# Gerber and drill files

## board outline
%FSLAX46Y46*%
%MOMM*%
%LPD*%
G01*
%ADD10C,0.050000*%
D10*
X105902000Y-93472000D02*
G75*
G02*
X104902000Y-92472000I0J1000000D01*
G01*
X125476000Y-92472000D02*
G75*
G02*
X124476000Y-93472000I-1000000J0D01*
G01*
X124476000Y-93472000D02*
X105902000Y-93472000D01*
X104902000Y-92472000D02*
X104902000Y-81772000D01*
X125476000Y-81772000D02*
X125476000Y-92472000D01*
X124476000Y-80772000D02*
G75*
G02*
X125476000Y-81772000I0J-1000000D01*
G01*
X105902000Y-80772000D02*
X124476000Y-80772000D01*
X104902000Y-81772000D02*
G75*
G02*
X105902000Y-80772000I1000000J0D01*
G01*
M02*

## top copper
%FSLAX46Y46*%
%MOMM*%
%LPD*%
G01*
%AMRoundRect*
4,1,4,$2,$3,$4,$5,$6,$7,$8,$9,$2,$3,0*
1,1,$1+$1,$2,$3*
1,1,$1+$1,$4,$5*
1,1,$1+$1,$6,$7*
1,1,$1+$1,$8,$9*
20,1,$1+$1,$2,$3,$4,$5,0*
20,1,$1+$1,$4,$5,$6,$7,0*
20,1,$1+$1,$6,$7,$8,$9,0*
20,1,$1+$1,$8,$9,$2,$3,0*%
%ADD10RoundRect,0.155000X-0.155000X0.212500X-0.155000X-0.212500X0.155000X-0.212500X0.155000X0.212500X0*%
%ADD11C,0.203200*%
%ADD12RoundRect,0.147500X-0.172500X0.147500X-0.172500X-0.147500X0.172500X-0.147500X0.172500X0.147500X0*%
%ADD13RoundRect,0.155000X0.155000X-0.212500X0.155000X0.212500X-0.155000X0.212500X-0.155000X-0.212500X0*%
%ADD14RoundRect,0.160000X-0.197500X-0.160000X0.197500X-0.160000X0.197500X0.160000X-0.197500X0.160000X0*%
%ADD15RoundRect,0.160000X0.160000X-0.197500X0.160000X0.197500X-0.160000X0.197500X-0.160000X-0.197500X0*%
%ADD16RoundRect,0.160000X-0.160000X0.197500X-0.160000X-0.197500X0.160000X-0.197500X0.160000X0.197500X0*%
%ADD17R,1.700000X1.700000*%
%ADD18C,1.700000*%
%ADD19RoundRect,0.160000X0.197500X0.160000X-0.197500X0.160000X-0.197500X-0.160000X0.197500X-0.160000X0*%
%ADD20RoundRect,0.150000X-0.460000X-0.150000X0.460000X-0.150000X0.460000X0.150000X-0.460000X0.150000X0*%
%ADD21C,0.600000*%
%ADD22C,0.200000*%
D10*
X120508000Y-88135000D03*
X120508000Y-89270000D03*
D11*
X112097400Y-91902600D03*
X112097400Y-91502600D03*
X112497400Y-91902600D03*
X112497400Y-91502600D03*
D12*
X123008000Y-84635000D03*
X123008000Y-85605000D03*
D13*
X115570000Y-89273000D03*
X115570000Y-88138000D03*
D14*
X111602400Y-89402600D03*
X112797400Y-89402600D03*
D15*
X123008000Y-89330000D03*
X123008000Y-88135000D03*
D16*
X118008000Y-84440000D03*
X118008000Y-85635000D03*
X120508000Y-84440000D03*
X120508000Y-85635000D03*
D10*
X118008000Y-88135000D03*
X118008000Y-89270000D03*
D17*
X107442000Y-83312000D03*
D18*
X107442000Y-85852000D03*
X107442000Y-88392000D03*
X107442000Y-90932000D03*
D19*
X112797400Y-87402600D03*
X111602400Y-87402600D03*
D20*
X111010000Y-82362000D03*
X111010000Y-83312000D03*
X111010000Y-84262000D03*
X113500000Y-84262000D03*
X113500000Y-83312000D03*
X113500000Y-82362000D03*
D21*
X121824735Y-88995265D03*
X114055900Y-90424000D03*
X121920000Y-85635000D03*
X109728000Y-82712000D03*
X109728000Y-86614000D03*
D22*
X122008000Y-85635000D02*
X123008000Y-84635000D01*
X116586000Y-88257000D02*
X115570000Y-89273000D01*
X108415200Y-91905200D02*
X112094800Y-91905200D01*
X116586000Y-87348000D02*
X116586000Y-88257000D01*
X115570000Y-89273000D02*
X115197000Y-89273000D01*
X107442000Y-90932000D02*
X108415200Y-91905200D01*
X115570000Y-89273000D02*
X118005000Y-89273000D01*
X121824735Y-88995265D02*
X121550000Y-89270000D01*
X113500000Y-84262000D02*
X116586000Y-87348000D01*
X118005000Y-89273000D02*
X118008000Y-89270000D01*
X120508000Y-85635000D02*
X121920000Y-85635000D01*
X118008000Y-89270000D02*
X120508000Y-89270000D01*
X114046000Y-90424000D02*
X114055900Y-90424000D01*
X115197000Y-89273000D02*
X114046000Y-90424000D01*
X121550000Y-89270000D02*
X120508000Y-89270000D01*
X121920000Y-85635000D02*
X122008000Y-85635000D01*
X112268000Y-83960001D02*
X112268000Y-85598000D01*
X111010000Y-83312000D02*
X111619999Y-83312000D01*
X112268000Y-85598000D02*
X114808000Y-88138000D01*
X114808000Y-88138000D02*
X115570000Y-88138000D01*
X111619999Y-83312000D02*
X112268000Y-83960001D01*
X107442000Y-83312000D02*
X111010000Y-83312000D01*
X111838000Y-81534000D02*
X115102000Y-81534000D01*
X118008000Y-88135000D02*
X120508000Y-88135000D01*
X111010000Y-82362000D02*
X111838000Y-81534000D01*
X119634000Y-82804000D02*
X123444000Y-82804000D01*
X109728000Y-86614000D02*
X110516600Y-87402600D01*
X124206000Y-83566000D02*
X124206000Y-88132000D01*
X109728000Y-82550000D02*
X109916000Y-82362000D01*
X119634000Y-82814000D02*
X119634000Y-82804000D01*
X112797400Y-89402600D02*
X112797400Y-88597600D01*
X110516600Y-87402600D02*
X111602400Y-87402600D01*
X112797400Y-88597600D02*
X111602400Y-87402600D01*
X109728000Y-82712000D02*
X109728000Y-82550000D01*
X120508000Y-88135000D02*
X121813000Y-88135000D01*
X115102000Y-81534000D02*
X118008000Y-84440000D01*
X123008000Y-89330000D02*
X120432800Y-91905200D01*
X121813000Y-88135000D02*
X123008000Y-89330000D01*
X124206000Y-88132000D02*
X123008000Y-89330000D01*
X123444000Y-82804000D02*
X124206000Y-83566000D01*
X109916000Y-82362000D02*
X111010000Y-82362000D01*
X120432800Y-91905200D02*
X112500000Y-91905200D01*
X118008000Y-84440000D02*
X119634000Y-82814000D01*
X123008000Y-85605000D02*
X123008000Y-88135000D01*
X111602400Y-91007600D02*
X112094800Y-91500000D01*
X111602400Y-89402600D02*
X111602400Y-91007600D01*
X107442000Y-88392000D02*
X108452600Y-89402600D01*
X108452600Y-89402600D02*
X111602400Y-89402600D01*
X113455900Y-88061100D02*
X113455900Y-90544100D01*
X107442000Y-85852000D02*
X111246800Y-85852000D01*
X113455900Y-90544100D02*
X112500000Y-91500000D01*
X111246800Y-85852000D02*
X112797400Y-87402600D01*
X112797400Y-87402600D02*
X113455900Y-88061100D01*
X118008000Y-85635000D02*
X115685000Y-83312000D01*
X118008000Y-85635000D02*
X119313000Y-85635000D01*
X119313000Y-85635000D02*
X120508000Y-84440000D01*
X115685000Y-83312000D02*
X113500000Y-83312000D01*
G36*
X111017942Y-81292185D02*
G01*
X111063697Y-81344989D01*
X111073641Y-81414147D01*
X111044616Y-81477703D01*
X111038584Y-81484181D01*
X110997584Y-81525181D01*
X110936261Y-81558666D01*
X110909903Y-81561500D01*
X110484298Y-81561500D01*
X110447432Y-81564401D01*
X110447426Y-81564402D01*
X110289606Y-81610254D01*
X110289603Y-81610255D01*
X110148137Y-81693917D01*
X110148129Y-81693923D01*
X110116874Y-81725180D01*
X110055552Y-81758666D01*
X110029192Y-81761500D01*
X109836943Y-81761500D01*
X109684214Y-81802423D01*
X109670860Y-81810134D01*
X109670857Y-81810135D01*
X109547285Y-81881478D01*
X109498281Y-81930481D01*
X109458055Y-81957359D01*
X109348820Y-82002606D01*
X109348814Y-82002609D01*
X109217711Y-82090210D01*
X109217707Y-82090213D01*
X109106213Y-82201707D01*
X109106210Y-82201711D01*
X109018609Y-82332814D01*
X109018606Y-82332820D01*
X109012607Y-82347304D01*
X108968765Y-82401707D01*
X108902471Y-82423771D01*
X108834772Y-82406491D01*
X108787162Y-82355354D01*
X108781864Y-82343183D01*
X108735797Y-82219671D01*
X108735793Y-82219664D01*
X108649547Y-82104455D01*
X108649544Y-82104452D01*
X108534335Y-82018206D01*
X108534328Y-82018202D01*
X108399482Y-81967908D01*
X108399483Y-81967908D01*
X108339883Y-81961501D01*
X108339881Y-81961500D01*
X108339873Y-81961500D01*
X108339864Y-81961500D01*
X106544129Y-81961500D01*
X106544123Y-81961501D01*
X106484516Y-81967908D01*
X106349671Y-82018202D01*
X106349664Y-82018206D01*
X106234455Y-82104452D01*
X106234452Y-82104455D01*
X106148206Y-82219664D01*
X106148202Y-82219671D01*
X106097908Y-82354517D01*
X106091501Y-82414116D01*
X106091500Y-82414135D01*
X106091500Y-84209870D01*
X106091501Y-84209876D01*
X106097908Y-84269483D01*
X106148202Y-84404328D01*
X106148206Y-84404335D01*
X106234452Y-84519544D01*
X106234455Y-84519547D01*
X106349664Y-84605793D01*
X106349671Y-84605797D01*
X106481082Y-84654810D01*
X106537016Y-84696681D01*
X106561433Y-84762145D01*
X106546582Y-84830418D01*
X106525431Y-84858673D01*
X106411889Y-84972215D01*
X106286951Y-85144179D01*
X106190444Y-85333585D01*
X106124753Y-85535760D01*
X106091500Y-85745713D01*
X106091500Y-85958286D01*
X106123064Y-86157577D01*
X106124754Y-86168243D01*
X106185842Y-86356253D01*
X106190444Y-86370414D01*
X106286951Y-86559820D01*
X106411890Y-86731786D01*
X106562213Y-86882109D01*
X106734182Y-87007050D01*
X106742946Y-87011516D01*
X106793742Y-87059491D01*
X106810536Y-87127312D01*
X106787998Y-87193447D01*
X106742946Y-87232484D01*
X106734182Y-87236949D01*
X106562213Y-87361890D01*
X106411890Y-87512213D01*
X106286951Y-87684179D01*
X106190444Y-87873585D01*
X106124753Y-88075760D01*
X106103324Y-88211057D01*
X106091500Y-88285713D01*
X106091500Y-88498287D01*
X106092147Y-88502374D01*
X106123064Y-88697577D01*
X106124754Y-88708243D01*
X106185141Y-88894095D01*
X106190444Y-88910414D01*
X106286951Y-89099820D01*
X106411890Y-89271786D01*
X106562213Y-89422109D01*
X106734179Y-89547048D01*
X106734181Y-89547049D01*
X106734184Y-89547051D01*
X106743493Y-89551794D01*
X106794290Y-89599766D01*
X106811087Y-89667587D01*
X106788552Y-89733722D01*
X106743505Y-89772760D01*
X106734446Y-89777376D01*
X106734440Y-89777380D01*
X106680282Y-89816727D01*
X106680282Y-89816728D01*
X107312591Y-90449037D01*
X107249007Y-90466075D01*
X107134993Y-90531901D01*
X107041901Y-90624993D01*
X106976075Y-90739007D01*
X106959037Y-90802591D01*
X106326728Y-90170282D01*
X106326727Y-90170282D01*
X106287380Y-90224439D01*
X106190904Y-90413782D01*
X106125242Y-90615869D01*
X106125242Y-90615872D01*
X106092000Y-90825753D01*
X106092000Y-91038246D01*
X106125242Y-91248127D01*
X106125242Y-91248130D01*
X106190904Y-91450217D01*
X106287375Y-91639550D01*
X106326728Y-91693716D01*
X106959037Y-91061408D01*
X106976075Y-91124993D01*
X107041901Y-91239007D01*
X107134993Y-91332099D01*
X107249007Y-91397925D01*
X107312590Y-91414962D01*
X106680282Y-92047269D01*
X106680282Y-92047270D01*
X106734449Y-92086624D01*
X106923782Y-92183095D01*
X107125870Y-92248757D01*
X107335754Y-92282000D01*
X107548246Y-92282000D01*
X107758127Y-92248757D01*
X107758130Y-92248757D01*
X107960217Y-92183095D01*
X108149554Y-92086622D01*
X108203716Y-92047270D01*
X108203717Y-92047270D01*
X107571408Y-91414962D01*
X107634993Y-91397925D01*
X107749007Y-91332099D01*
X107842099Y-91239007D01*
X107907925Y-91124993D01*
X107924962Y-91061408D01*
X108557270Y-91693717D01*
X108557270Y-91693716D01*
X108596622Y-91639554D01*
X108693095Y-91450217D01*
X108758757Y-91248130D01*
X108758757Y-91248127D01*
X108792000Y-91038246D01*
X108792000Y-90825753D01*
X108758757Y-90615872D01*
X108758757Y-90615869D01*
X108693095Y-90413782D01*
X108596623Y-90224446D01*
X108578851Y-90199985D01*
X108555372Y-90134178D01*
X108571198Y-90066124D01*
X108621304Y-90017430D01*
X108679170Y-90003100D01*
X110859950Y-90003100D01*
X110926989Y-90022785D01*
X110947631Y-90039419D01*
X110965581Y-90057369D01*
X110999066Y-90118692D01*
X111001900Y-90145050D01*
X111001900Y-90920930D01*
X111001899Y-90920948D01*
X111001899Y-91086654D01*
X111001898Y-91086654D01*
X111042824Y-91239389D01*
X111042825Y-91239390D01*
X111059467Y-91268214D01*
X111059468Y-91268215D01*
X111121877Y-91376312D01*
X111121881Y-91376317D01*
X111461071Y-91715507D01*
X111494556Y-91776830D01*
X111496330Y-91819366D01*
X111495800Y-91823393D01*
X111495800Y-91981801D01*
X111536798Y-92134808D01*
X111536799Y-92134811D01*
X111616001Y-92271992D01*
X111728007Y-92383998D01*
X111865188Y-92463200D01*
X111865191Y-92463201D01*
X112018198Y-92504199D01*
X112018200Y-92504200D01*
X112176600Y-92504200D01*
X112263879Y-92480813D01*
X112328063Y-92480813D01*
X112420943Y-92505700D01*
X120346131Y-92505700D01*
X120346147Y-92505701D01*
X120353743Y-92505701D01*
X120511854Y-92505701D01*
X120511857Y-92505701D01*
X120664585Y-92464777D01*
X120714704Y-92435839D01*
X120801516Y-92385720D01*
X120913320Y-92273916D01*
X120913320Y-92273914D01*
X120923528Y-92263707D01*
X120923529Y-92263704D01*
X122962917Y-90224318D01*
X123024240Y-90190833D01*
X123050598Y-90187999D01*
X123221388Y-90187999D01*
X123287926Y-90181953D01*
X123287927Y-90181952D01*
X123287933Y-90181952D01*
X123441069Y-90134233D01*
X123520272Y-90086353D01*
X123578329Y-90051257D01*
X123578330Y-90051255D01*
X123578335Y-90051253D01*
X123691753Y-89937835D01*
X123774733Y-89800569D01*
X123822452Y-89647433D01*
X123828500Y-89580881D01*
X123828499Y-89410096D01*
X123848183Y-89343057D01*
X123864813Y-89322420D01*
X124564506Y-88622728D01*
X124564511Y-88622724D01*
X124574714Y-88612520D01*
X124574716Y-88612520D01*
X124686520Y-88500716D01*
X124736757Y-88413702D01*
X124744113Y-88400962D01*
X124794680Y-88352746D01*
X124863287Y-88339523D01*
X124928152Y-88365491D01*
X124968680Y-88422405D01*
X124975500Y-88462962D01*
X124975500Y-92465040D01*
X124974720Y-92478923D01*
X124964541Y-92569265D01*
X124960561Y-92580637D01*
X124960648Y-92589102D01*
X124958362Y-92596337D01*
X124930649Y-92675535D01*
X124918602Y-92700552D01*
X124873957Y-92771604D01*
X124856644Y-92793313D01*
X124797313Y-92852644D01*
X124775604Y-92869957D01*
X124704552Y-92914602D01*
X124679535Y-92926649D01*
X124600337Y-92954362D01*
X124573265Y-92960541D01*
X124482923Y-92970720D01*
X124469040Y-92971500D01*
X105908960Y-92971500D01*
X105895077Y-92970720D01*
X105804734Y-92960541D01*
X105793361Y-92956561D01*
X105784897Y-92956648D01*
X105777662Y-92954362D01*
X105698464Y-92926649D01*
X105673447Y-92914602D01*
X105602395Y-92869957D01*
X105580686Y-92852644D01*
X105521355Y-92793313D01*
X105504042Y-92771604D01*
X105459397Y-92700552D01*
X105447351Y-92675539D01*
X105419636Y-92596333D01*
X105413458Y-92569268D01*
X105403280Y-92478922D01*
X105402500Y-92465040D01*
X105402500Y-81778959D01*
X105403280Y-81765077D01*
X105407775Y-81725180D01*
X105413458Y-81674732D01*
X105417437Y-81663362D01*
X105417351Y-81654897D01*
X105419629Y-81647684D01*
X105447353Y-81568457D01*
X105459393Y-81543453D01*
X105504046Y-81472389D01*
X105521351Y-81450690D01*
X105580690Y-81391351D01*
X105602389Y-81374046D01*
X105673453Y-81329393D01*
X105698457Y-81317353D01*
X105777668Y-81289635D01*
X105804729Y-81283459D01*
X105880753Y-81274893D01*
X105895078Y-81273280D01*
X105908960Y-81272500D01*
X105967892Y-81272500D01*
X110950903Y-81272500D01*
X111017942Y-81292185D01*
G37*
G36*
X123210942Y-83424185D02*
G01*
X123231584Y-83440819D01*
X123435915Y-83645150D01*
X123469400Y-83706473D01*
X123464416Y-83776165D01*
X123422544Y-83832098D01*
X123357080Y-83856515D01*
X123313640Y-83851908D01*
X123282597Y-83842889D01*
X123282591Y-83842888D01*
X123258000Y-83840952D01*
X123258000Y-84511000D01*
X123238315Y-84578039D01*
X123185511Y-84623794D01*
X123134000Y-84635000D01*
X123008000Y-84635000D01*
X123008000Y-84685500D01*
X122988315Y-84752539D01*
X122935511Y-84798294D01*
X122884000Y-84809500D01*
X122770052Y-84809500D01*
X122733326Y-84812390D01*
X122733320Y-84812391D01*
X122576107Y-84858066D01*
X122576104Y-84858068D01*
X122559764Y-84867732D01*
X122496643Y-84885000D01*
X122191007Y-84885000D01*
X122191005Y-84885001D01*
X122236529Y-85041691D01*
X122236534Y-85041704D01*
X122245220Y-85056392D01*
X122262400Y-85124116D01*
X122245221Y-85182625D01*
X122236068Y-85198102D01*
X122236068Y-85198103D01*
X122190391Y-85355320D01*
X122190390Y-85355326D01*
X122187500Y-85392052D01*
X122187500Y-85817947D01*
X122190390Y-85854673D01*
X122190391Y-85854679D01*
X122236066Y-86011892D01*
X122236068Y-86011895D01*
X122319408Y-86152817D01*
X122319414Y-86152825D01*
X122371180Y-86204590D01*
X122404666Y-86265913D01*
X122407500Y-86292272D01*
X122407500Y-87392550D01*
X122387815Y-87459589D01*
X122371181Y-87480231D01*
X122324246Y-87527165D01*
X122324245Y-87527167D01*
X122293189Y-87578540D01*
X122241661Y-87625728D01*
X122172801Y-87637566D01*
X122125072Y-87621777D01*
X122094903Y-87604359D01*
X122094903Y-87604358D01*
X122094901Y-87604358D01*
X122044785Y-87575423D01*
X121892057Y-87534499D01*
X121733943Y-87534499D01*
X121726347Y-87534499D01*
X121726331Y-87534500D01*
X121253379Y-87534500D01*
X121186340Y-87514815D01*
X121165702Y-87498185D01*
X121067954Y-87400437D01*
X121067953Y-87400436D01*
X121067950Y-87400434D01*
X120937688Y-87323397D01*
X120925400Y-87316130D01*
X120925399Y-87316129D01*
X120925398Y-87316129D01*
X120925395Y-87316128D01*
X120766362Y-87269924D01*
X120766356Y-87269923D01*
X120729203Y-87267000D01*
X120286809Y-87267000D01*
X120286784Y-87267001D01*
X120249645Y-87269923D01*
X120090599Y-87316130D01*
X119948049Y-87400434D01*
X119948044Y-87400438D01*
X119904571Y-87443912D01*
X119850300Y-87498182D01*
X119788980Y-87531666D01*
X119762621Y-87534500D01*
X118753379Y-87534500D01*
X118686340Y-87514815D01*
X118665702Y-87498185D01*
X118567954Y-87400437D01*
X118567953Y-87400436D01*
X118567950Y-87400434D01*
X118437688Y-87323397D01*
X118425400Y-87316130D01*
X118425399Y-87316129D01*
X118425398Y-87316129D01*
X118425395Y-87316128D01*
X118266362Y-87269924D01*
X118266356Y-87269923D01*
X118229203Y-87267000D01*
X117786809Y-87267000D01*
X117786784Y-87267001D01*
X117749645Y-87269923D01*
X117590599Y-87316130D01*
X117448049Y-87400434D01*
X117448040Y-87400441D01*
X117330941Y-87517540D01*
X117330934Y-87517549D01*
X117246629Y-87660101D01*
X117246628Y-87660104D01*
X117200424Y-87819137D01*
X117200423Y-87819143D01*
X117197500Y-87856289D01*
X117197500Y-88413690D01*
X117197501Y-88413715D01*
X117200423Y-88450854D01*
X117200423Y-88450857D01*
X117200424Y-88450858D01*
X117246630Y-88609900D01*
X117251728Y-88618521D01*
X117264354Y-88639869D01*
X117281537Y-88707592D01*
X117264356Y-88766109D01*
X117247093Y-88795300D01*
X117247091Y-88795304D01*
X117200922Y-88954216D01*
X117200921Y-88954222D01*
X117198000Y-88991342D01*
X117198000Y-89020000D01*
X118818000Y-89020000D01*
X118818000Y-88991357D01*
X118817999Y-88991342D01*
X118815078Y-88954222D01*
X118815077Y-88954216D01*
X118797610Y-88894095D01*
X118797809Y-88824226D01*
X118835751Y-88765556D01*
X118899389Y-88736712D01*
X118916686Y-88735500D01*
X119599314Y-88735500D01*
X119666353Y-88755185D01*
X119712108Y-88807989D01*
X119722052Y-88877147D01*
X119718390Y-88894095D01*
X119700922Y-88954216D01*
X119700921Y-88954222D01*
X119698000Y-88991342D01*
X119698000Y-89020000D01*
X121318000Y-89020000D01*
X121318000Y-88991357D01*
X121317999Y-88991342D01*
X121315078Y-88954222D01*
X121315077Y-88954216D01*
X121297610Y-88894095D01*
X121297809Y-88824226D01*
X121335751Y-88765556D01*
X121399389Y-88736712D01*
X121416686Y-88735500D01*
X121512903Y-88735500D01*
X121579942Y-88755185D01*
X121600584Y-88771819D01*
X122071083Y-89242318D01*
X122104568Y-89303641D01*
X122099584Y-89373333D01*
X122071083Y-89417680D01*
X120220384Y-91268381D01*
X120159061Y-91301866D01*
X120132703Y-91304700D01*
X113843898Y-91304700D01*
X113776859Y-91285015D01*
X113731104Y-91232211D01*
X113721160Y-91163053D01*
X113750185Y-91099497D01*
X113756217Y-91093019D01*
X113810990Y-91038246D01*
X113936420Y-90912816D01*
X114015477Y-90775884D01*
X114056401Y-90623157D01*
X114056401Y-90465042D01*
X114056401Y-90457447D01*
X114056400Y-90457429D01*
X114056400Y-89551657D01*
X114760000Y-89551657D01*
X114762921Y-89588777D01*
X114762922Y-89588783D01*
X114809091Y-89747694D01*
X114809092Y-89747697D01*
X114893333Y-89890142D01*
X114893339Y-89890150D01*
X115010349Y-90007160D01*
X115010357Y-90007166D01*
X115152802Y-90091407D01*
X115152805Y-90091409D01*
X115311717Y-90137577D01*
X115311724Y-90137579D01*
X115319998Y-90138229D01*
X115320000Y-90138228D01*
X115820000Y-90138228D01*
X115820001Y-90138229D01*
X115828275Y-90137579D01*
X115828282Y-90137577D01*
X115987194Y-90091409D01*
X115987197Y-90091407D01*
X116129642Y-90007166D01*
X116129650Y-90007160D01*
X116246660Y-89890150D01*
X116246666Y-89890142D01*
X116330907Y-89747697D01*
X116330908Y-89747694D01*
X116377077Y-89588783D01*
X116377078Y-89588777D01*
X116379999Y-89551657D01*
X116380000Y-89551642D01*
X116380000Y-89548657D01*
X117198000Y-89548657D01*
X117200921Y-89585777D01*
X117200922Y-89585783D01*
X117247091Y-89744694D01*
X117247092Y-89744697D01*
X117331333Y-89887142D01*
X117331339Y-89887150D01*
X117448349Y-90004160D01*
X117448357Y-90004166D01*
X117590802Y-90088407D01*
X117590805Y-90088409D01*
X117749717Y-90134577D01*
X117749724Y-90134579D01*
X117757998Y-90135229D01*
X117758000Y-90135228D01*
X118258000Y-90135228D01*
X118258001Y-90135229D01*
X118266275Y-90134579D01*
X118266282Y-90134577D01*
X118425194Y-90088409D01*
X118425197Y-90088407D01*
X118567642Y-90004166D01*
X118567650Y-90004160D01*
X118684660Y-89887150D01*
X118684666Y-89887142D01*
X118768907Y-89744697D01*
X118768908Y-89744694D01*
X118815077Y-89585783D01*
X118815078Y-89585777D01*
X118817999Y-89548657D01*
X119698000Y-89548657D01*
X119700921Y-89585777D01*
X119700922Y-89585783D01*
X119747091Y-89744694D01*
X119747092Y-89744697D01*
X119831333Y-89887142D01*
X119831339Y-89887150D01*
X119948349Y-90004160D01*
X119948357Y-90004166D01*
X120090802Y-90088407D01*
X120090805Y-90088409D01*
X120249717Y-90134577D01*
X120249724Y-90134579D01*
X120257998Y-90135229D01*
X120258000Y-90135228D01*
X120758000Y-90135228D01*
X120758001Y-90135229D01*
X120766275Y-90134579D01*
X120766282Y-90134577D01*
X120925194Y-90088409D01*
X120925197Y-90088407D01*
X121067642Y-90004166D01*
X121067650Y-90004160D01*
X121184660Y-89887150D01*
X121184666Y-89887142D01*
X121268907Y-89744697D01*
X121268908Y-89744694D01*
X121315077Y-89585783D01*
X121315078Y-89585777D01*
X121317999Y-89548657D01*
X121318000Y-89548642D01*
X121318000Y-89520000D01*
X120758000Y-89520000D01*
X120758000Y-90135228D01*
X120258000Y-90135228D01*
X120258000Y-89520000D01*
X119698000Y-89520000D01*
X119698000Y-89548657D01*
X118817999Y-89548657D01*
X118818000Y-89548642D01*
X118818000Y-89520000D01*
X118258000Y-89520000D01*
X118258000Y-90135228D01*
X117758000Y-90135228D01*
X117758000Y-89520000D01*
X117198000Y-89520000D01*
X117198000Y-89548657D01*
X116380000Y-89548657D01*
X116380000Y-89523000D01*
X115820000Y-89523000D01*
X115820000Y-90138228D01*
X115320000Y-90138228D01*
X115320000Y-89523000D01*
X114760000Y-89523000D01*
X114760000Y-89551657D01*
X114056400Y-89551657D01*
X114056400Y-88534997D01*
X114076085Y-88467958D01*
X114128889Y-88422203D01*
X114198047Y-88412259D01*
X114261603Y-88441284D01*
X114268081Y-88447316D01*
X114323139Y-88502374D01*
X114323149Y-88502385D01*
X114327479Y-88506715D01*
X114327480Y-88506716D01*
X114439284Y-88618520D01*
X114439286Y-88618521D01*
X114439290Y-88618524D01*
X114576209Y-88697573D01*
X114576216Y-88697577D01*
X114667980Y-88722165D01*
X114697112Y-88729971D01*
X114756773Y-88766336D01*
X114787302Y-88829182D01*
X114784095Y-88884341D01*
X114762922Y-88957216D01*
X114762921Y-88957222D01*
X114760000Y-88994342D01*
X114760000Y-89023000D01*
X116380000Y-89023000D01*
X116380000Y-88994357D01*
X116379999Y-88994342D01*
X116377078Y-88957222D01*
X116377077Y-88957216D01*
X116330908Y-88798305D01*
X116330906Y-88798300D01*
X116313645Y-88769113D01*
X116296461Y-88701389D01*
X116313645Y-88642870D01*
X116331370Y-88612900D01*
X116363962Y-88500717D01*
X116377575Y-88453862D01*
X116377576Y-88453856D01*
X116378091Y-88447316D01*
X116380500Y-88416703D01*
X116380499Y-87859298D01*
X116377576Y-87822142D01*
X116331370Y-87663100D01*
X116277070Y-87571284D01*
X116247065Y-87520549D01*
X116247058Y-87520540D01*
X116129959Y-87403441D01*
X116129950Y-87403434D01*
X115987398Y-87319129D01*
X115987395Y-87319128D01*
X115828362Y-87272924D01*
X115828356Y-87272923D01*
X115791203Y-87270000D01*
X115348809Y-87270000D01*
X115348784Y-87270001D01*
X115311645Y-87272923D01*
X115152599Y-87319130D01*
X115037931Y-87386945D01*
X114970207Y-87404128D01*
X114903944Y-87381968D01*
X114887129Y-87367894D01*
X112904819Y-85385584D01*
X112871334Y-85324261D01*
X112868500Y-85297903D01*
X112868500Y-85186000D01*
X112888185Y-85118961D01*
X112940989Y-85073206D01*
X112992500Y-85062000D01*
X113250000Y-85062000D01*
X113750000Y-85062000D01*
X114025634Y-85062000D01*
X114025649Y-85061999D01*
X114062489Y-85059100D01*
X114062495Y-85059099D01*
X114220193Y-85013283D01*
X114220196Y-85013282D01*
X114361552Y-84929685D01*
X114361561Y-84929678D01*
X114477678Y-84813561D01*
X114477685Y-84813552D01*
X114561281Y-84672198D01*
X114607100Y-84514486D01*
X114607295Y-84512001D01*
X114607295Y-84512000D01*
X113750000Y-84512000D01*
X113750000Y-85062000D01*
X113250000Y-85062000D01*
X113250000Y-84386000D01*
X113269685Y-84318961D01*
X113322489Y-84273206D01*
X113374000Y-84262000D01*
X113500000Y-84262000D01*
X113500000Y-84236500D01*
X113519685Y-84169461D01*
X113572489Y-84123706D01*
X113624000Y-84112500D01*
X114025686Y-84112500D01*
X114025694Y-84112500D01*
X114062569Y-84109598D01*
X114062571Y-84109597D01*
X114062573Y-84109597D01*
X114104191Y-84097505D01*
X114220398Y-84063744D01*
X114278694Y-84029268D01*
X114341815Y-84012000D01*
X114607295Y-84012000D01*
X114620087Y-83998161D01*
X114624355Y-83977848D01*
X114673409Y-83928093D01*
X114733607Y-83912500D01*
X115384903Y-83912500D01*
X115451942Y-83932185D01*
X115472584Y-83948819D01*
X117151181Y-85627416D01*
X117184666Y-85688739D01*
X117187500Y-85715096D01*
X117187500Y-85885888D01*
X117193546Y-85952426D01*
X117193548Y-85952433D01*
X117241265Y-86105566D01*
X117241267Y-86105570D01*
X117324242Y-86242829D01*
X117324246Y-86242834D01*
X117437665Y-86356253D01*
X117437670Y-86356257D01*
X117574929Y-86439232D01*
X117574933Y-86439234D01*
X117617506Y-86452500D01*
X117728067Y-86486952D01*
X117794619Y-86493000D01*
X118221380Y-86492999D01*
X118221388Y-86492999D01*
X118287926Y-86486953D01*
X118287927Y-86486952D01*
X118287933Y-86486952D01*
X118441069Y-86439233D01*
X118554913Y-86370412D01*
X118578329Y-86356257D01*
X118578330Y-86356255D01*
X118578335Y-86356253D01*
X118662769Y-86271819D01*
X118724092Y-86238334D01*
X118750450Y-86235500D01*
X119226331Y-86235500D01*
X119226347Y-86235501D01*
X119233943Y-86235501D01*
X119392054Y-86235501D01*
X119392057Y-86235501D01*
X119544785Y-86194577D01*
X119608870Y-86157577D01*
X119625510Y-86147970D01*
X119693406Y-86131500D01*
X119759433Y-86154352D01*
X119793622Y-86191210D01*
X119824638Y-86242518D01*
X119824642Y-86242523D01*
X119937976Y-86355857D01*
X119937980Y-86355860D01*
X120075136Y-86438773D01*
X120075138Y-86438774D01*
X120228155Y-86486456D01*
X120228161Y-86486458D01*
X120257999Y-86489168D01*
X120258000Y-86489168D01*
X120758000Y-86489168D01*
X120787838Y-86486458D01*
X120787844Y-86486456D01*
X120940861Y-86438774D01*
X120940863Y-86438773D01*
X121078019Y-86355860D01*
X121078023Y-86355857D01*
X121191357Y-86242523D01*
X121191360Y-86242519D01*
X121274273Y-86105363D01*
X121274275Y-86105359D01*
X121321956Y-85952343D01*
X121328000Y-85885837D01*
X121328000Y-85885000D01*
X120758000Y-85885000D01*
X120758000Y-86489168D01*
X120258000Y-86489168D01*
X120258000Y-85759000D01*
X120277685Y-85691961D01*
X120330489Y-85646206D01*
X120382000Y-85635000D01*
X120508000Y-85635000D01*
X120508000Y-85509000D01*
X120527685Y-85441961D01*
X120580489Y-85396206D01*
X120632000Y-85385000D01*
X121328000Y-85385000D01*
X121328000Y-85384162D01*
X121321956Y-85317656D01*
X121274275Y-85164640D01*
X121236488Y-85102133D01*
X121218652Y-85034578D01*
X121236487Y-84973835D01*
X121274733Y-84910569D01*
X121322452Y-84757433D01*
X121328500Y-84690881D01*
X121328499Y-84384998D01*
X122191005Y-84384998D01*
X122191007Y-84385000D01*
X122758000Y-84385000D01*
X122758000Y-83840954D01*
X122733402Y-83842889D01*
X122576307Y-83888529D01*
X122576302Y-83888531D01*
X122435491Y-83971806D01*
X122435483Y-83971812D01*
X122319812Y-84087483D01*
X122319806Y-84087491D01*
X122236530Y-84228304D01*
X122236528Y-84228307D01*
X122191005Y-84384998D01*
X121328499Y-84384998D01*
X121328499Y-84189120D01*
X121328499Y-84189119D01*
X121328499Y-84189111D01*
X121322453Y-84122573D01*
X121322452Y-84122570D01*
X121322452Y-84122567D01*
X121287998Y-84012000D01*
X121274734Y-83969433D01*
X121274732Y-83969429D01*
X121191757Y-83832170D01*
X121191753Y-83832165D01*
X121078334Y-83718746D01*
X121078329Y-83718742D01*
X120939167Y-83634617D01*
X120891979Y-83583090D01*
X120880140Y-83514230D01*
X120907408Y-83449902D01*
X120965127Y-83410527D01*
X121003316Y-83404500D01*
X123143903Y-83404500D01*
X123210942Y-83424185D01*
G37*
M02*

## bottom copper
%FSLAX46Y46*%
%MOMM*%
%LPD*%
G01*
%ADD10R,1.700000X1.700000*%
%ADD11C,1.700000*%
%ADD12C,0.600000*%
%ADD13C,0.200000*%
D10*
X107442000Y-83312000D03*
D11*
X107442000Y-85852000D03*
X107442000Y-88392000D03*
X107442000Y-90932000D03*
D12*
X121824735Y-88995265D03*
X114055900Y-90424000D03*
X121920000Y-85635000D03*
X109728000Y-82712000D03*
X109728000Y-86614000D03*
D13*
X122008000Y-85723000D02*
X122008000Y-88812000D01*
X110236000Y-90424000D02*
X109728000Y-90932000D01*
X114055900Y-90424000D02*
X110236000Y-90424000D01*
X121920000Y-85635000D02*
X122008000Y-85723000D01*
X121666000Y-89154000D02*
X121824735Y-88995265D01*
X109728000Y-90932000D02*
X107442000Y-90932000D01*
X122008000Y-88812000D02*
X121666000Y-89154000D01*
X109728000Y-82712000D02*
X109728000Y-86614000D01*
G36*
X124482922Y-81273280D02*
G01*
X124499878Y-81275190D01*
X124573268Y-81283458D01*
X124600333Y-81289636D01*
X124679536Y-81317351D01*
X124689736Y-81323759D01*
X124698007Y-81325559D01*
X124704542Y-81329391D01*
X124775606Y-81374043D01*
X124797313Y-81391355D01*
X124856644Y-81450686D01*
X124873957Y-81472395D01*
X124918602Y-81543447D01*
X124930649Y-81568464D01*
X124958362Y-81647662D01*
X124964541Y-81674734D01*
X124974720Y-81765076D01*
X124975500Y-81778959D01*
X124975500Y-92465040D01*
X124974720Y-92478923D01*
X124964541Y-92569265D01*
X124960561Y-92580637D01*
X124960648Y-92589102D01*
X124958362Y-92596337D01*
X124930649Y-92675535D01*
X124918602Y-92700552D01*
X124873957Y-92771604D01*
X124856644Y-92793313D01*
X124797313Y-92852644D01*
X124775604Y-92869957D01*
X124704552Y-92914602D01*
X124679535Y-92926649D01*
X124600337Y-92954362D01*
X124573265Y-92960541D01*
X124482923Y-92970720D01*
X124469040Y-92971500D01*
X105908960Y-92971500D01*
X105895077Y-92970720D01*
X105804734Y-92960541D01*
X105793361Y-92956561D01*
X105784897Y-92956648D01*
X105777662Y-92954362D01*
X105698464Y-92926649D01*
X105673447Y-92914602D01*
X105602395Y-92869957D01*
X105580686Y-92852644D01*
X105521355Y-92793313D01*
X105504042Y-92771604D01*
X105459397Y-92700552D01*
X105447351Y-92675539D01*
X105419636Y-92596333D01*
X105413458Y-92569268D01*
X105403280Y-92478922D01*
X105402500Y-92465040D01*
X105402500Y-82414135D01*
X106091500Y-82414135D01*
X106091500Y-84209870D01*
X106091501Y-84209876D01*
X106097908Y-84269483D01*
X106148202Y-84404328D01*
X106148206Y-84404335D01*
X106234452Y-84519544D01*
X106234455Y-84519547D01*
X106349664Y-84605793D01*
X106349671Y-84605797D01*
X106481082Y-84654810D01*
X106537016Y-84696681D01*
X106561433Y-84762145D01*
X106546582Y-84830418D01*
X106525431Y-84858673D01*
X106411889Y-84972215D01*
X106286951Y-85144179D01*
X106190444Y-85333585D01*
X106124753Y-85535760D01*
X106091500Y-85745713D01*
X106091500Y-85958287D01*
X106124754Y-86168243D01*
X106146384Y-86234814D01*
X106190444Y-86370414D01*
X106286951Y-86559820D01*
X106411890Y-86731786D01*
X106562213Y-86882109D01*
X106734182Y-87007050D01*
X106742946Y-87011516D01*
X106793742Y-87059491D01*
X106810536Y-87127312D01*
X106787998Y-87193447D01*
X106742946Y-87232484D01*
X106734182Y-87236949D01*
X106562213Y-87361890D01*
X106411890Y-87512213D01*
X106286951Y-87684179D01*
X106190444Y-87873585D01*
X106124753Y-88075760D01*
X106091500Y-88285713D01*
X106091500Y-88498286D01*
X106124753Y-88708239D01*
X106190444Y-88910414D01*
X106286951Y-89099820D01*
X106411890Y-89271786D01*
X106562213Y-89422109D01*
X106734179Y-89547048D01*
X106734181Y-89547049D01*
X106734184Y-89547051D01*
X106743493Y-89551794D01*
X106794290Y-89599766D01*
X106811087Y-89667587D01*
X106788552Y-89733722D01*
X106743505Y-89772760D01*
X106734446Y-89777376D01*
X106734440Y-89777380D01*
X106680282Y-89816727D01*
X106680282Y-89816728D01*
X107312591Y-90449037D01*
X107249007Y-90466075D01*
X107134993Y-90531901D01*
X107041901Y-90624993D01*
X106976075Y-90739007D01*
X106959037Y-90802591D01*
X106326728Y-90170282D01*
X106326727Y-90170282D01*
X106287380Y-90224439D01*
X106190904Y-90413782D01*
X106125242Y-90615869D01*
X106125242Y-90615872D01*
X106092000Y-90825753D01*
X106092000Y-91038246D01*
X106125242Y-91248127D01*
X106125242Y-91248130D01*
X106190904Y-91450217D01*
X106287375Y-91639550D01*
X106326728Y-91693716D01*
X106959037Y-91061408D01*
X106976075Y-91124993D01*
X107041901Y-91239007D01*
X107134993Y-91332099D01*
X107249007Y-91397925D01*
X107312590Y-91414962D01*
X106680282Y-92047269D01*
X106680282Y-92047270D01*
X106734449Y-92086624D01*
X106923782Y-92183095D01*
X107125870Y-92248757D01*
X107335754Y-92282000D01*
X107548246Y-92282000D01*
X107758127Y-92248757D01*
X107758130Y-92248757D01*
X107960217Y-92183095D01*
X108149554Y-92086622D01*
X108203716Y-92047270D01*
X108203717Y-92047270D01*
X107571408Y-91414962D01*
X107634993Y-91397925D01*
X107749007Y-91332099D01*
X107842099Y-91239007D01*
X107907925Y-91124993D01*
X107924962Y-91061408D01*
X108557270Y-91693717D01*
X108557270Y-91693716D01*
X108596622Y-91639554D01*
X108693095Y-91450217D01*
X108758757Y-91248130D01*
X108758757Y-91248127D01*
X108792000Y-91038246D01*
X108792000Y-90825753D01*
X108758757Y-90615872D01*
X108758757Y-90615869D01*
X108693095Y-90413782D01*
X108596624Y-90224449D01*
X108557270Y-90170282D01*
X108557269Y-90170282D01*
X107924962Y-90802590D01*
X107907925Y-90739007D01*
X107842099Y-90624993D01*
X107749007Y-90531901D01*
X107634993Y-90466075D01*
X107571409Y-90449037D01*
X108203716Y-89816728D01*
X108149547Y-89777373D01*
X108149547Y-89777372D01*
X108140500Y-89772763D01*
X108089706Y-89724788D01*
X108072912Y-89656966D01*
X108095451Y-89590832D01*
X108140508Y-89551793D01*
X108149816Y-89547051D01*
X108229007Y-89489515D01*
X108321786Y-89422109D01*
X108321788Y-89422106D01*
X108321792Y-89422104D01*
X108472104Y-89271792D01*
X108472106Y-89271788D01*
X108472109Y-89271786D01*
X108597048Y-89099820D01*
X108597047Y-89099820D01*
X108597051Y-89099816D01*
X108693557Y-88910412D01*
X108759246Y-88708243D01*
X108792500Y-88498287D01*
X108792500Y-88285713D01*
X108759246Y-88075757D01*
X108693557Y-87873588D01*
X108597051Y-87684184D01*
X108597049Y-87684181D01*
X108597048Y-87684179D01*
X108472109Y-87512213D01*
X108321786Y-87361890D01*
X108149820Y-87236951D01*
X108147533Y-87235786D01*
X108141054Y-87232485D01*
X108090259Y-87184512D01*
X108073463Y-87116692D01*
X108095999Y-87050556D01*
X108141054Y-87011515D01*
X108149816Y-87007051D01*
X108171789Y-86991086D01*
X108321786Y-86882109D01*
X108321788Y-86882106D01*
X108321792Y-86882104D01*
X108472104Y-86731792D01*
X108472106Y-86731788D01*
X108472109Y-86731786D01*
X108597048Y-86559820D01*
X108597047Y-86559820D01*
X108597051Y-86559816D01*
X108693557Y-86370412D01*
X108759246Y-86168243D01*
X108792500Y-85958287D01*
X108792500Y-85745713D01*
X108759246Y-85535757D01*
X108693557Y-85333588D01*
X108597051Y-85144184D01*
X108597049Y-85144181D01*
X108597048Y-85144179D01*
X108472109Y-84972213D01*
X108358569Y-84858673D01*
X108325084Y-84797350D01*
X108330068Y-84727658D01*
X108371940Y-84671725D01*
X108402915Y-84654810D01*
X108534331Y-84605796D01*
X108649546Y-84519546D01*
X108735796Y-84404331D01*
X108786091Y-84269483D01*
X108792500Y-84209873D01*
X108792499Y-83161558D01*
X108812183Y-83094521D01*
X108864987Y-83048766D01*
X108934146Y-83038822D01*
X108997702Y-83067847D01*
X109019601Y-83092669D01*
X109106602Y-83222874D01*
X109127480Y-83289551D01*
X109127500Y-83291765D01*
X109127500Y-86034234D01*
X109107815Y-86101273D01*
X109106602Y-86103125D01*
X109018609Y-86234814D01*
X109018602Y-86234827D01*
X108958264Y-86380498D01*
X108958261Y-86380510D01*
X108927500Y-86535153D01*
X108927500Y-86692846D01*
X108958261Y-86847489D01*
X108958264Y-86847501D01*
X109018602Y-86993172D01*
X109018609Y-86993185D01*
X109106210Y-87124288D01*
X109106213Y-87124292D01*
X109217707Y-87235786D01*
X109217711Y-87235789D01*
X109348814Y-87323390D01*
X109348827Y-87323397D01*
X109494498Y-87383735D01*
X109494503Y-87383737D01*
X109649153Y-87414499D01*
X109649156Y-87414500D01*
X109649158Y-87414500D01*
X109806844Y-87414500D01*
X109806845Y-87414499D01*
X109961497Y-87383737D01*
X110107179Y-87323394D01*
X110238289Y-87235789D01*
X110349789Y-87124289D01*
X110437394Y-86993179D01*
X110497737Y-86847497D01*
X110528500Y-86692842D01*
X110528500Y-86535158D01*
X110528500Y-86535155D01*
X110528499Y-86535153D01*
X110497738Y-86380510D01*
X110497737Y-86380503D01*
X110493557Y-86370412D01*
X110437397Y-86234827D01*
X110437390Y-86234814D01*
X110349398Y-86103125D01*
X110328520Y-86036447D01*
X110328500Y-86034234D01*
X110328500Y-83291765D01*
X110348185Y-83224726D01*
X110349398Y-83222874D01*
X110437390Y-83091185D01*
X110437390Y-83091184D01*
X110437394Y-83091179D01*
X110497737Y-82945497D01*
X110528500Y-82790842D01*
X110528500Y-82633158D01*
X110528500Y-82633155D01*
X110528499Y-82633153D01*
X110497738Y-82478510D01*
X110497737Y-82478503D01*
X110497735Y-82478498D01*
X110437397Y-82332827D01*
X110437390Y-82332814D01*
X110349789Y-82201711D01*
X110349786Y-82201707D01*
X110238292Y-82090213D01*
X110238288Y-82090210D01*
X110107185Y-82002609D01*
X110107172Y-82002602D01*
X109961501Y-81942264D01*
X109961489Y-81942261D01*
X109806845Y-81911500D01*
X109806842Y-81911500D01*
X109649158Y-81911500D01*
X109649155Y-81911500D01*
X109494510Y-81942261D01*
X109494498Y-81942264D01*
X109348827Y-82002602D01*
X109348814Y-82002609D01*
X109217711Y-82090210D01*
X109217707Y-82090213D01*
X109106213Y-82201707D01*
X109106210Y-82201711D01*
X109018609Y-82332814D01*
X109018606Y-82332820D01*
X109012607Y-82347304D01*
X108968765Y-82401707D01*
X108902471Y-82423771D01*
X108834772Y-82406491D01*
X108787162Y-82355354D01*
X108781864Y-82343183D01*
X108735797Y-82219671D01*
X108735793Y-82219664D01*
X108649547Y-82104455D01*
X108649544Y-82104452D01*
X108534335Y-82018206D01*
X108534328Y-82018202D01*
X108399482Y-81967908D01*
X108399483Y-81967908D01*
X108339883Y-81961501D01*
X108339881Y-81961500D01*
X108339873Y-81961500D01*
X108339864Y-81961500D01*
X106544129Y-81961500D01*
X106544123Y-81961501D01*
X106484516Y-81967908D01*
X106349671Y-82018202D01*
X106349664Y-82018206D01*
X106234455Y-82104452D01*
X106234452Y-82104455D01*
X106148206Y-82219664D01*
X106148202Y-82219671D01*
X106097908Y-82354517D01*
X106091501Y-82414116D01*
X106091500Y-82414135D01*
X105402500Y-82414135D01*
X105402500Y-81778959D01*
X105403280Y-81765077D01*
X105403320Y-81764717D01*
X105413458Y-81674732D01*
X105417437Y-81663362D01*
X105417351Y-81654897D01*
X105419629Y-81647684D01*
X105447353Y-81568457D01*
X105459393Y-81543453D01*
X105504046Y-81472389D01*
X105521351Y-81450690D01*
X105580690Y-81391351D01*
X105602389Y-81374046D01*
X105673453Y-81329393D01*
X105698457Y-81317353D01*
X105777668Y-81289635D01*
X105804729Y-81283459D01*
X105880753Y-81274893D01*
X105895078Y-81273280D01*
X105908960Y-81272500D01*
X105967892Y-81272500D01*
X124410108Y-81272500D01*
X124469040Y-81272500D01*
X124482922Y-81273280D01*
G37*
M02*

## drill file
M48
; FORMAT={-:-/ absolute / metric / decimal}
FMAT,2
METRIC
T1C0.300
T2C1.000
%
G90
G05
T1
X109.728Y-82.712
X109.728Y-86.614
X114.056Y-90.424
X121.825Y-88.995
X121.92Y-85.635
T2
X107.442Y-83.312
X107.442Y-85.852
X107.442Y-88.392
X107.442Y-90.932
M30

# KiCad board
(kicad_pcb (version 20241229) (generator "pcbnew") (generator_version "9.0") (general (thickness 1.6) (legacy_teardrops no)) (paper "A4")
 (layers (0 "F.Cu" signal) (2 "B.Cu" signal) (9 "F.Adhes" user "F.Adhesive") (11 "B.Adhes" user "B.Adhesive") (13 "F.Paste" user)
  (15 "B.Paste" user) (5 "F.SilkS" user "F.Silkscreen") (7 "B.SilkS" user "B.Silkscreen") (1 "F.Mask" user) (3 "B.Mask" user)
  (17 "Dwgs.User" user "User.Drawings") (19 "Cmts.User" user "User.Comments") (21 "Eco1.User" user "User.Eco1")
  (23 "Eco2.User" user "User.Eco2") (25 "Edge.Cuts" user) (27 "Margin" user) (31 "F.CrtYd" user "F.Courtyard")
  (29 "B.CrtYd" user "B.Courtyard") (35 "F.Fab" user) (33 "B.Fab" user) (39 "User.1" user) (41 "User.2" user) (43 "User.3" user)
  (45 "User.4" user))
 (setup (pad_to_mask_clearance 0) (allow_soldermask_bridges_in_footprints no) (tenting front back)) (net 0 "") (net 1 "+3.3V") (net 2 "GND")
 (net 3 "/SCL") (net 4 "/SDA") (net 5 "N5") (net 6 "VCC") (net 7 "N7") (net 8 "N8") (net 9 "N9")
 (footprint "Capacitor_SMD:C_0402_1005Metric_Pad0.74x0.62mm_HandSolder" (layer "F.Cu") (at 120.508 88.7025 -90)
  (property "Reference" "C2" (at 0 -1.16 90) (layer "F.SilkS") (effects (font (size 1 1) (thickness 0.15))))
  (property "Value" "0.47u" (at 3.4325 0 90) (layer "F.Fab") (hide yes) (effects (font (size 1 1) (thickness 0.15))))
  (pad "1" smd roundrect (at -0.5675 0 270) (size 0.735 0.62) (layers "F.Cu" "F.Mask" "F.Paste") (roundrect_rratio 0.25) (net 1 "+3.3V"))
  (pad "2" smd roundrect (at 0.5675 0 270) (size 0.735 0.62) (layers "F.Cu" "F.Mask" "F.Paste") (roundrect_rratio 0.25) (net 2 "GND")))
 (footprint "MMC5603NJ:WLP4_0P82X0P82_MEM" (layer "F.Cu") (at 112.2974 91.7026 90)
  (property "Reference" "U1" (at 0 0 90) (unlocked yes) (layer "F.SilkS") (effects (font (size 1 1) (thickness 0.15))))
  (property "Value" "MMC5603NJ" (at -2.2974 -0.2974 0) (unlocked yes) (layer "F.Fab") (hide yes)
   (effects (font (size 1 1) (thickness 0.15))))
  (pad "A1" smd circle (at -0.2 -0.2 90) (size 0.2032 0.2032) (layers "F.Cu" "F.Mask" "F.Paste") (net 2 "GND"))
  (pad "A2" smd circle (at 0.2 -0.2 90) (size 0.2032 0.2032) (layers "F.Cu" "F.Mask" "F.Paste") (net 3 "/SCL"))
  (pad "B1" smd circle (at -0.2 0.2 90) (size 0.2032 0.2032) (layers "F.Cu" "F.Mask" "F.Paste") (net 1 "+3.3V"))
  (pad "B2" smd circle (at 0.2 0.2 90) (size 0.2032 0.2032) (layers "F.Cu" "F.Mask" "F.Paste") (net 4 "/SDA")))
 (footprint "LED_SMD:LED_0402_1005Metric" (layer "F.Cu") (at 123.008 85.12 -90)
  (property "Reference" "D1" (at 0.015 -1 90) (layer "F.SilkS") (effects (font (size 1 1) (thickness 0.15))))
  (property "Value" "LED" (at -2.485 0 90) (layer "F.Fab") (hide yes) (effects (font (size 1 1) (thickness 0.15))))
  (pad "1" smd roundrect (at -0.485 0 270) (size 0.59 0.64) (layers "F.Cu" "F.Mask" "F.Paste") (roundrect_rratio 0.25) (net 2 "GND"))
  (pad "2" smd roundrect (at 0.485 0 270) (size 0.59 0.64) (layers "F.Cu" "F.Mask" "F.Paste") (roundrect_rratio 0.25) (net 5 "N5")))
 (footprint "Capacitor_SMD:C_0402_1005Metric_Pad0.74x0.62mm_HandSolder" (layer "F.Cu") (at 115.57 88.7055 90)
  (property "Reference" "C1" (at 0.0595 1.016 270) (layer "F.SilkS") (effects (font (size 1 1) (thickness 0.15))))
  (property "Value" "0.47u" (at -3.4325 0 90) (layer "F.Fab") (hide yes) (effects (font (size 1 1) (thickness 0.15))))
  (pad "1" smd roundrect (at -0.5675 0 90) (size 0.735 0.62) (layers "F.Cu" "F.Mask" "F.Paste") (roundrect_rratio 0.25) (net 2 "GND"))
  (pad "2" smd roundrect (at 0.5675 0 90) (size 0.735 0.62) (layers "F.Cu" "F.Mask" "F.Paste") (roundrect_rratio 0.25) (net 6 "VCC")))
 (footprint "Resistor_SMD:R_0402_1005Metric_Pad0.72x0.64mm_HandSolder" (layer "F.Cu") (at 112.1999 89.4026)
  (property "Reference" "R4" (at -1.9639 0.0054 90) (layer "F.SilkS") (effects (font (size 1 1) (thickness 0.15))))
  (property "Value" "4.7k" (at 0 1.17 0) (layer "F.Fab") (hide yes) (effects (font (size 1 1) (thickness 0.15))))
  (pad "1" smd roundrect (at -0.5975 0) (size 0.715 0.64) (layers "F.Cu" "F.Mask" "F.Paste") (roundrect_rratio 0.25) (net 3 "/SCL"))
  (pad "2" smd roundrect (at 0.5975 0) (size 0.715 0.64) (layers "F.Cu" "F.Mask" "F.Paste") (roundrect_rratio 0.25) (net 1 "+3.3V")))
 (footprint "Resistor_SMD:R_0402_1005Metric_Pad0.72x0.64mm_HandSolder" (layer "F.Cu") (at 123.008 88.7325 90)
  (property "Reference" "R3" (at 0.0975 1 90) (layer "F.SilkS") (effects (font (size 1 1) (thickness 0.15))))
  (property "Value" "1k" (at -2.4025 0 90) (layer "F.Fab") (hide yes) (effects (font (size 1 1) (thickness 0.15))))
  (pad "1" smd roundrect (at -0.5975 0 90) (size 0.715 0.64) (layers "F.Cu" "F.Mask" "F.Paste") (roundrect_rratio 0.25) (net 1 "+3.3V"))
  (pad "2" smd roundrect (at 0.5975 0 90) (size 0.715 0.64) (layers "F.Cu" "F.Mask" "F.Paste") (roundrect_rratio 0.25) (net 5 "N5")))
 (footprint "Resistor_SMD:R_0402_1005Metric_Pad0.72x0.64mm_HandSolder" (layer "F.Cu") (at 118.008 85.0375 -90)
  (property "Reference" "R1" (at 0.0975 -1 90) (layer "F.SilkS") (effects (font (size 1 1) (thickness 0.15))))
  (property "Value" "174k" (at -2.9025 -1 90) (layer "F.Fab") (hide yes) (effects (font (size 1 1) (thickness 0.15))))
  (pad "1" smd roundrect (at -0.5975 0 270) (size 0.715 0.64) (layers "F.Cu" "F.Mask" "F.Paste") (roundrect_rratio 0.25) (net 1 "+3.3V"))
  (pad "2" smd roundrect (at 0.5975 0 270) (size 0.715 0.64) (layers "F.Cu" "F.Mask" "F.Paste") (roundrect_rratio 0.25) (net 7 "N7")))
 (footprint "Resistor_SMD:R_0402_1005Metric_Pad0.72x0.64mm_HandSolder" (layer "F.Cu") (at 120.508 85.0375 -90)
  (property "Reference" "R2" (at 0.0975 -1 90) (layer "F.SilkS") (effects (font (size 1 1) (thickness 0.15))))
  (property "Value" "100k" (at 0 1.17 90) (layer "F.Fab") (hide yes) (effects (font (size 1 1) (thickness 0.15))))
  (pad "1" smd roundrect (at -0.5975 0 270) (size 0.715 0.64) (layers "F.Cu" "F.Mask" "F.Paste") (roundrect_rratio 0.25) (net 7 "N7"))
  (pad "2" smd roundrect (at 0.5975 0 270) (size 0.715 0.64) (layers "F.Cu" "F.Mask" "F.Paste") (roundrect_rratio 0.25) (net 2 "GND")))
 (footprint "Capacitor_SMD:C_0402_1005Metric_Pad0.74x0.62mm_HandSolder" (layer "F.Cu") (at 118.008 88.7025 -90)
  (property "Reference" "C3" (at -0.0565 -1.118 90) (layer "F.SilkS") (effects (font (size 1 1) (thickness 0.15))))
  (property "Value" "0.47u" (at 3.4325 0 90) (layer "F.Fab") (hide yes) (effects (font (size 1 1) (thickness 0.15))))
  (pad "1" smd roundrect (at -0.5675 0 270) (size 0.735 0.62) (layers "F.Cu" "F.Mask" "F.Paste") (roundrect_rratio 0.25) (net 1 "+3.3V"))
  (pad "2" smd roundrect (at 0.5675 0 270) (size 0.735 0.62) (layers "F.Cu" "F.Mask" "F.Paste") (roundrect_rratio 0.25) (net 2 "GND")))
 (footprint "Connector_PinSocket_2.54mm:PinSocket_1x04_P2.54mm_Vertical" (layer "F.Cu") (at 107.442 83.312)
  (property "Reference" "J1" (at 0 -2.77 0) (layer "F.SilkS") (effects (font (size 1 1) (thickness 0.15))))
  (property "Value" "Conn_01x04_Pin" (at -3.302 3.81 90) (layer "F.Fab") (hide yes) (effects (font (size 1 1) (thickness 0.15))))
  (pad "1" thru_hole rect (at 0 0) (size 1.7 1.7) (drill 1) (layers "*.Cu" "*.Mask") (remove_unused_layers no) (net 6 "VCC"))
  (pad "2" thru_hole circle (at 0 2.54) (size 1.7 1.7) (drill 1) (layers "*.Cu" "*.Mask") (remove_unused_layers no) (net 4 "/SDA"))
  (pad "3" thru_hole circle (at 0 5.08) (size 1.7 1.7) (drill 1) (layers "*.Cu" "*.Mask") (remove_unused_layers no) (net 3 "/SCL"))
  (pad "4" thru_hole circle (at 0 7.62) (size 1.7 1.7) (drill 1) (layers "*.Cu" "*.Mask") (remove_unused_layers no) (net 2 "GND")))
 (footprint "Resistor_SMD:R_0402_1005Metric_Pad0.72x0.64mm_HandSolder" (layer "F.Cu") (at 112.1999 87.4026 180)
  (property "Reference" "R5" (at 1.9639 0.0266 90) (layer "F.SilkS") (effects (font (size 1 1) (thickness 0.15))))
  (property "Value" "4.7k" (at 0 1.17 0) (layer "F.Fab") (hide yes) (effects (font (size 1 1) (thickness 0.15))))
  (pad "1" smd roundrect (at -0.5975 0 180) (size 0.715 0.64) (layers "F.Cu" "F.Mask" "F.Paste") (roundrect_rratio 0.25) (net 4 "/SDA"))
  (pad "2" smd roundrect (at 0.5975 0 180) (size 0.715 0.64) (layers "F.Cu" "F.Mask" "F.Paste") (roundrect_rratio 0.25) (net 1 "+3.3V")))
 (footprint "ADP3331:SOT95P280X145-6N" (layer "F.Cu") (at 112.255 83.312)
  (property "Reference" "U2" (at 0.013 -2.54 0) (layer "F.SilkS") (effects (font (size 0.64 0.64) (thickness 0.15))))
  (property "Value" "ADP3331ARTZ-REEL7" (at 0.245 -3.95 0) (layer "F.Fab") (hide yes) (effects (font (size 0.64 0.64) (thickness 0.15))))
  (pad "1" smd roundrect (at -1.245 -0.95) (size 1.22 0.6) (layers "F.Cu" "F.Mask" "F.Paste") (roundrect_rratio 0.25) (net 1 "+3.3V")
   (solder_mask_margin 0.102))
  (pad "2" smd roundrect (at -1.245 0) (size 1.22 0.6) (layers "F.Cu" "F.Mask" "F.Paste") (roundrect_rratio 0.25) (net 6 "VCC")
   (solder_mask_margin 0.102))
  (pad "3" smd roundrect (at -1.245 0.95) (size 1.22 0.6) (layers "F.Cu" "F.Mask" "F.Paste") (roundrect_rratio 0.25) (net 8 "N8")
   (solder_mask_margin 0.102))
  (pad "4" smd roundrect (at 1.245 0.95) (size 1.22 0.6) (layers "F.Cu" "F.Mask" "F.Paste") (roundrect_rratio 0.25) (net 2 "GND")
   (solder_mask_margin 0.102))
  (pad "5" smd roundrect (at 1.245 0) (size 1.22 0.6) (layers "F.Cu" "F.Mask" "F.Paste") (roundrect_rratio 0.25) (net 7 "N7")
   (solder_mask_margin 0.102))
  (pad "6" smd roundrect (at 1.245 -0.95) (size 1.22 0.6) (layers "F.Cu" "F.Mask" "F.Paste") (roundrect_rratio 0.25) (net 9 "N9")
   (solder_mask_margin 0.102)))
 (gr_arc (start 105.902 93.472) (mid 105.194893 93.179107) (end 104.902 92.472) (stroke (width 0.05) (type default)) (layer "Edge.Cuts"))
 (gr_arc (start 125.476 92.472) (mid 125.183107 93.179107) (end 124.476 93.472) (stroke (width 0.05) (type default)) (layer "Edge.Cuts"))
 (gr_line (start 124.476 93.472) (end 105.902 93.472) (stroke (width 0.05) (type default)) (layer "Edge.Cuts"))
 (gr_line (start 104.902 92.472) (end 104.902 81.772) (stroke (width 0.05) (type default)) (layer "Edge.Cuts"))
 (gr_line (start 125.476 81.772) (end 125.476 92.472) (stroke (width 0.05) (type default)) (layer "Edge.Cuts"))
 (gr_arc (start 124.476 80.772) (mid 125.183107 81.064893) (end 125.476 81.772) (stroke (width 0.05) (type default)) (layer "Edge.Cuts"))
 (gr_line (start 105.902 80.772) (end 124.476 80.772) (stroke (width 0.05) (type default)) (layer "Edge.Cuts"))
 (gr_arc (start 104.902 81.772) (mid 105.194893 81.064893) (end 105.902 80.772) (stroke (width 0.05) (type default)) (layer "Edge.Cuts"))
 (segment (start 122.008 85.635) (end 123.008 84.635) (width 0.2) (layer "F.Cu") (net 2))
 (segment (start 116.586 88.257) (end 115.57 89.273) (width 0.2) (layer "F.Cu") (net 2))
 (segment (start 108.4152 91.9052) (end 112.0948 91.9052) (width 0.2) (layer "F.Cu") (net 2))
 (segment (start 116.586 87.348) (end 116.586 88.257) (width 0.2) (layer "F.Cu") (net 2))
 (segment (start 115.57 89.273) (end 115.197 89.273) (width 0.2) (layer "F.Cu") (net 2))
 (segment (start 107.442 90.932) (end 108.4152 91.9052) (width 0.2) (layer "F.Cu") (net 2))
 (segment (start 115.57 89.273) (end 118.005 89.273) (width 0.2) (layer "F.Cu") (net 2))
 (segment (start 121.824735 88.995265) (end 121.55 89.27) (width 0.2) (layer "F.Cu") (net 2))
 (segment (start 113.5 84.262) (end 116.586 87.348) (width 0.2) (layer "F.Cu") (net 2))
 (segment (start 118.005 89.273) (end 118.008 89.27) (width 0.2) (layer "F.Cu") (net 2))
 (segment (start 120.508 85.635) (end 121.92 85.635) (width 0.2) (layer "F.Cu") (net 2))
 (segment (start 118.008 89.27) (end 120.508 89.27) (width 0.2) (layer "F.Cu") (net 2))
 (segment (start 114.046 90.424) (end 114.0559 90.424) (width 0.2) (layer "F.Cu") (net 2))
 (segment (start 115.197 89.273) (end 114.046 90.424) (width 0.2) (layer "F.Cu") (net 2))
 (segment (start 121.55 89.27) (end 120.508 89.27) (width 0.2) (layer "F.Cu") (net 2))
 (segment (start 121.92 85.635) (end 122.008 85.635) (width 0.2) (layer "F.Cu") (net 2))
 (via (at 121.824735 88.995265) (size 0.6) (drill 0.3) (layers "F.Cu" "B.Cu") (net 2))
 (via (at 114.0559 90.424) (size 0.6) (drill 0.3) (layers "F.Cu" "B.Cu") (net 2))
 (via (at 121.92 85.635) (size 0.6) (drill 0.3) (layers "F.Cu" "B.Cu") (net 2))
 (segment (start 122.008 85.723) (end 122.008 88.812) (width 0.2) (layer "B.Cu") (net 2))
 (segment (start 110.236 90.424) (end 109.728 90.932) (width 0.2) (layer "B.Cu") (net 2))
 (segment (start 114.0559 90.424) (end 110.236 90.424) (width 0.2) (layer "B.Cu") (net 2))
 (segment (start 121.92 85.635) (end 122.008 85.723) (width 0.2) (layer "B.Cu") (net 2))
 (segment (start 121.666 89.154) (end 121.824735 88.995265) (width 0.2) (layer "B.Cu") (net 2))
 (segment (start 109.728 90.932) (end 107.442 90.932) (width 0.2) (layer "B.Cu") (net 2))
 (segment (start 122.008 88.812) (end 121.666 89.154) (width 0.2) (layer "B.Cu") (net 2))
 (segment (start 112.268 83.960001) (end 112.268 85.598) (width 0.2) (layer "F.Cu") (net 6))
 (segment (start 111.01 83.312) (end 111.619999 83.312) (width 0.2) (layer "F.Cu") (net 6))
 (segment (start 112.268 85.598) (end 114.808 88.138) (width 0.2) (layer "F.Cu") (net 6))
 (segment (start 114.808 88.138) (end 115.57 88.138) (width 0.2) (layer "F.Cu") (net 6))
 (segment (start 111.619999 83.312) (end 112.268 83.960001) (width 0.2) (layer "F.Cu") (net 6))
 (segment (start 107.442 83.312) (end 111.01 83.312) (width 0.2) (layer "F.Cu") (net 6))
 (segment (start 111.838 81.534) (end 115.102 81.534) (width 0.2) (layer "F.Cu") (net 1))
 (segment (start 118.008 88.135) (end 120.508 88.135) (width 0.2) (layer "F.Cu") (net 1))
 (segment (start 111.01 82.362) (end 111.838 81.534) (width 0.2) (layer "F.Cu") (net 1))
 (segment (start 119.634 82.804) (end 123.444 82.804) (width 0.2) (layer "F.Cu") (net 1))
 (segment (start 109.728 86.614) (end 110.5166 87.4026) (width 0.2) (layer "F.Cu") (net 1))
 (segment (start 124.206 83.566) (end 124.206 88.132) (width 0.2) (layer "F.Cu") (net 1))
 (segment (start 109.728 82.55) (end 109.916 82.362) (width 0.2) (layer "F.Cu") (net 1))
 (segment (start 119.634 82.814) (end 119.634 82.804) (width 0.2) (layer "F.Cu") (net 1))
 (segment (start 112.7974 89.4026) (end 112.7974 88.5976) (width 0.2) (layer "F.Cu") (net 1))
 (segment (start 110.5166 87.4026) (end 111.6024 87.4026) (width 0.2) (layer "F.Cu") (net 1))
 (segment (start 112.7974 88.5976) (end 111.6024 87.4026) (width 0.2) (layer "F.Cu") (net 1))
 (segment (start 109.728 82.712) (end 109.728 82.55) (width 0.2) (layer "F.Cu") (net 1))
 (segment (start 120.508 88.135) (end 121.813 88.135) (width 0.2) (layer "F.Cu") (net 1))
 (segment (start 115.102 81.534) (end 118.008 84.44) (width 0.2) (layer "F.Cu") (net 1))
 (segment (start 123.008 89.33) (end 120.4328 91.9052) (width 0.2) (layer "F.Cu") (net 1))
 (segment (start 121.813 88.135) (end 123.008 89.33) (width 0.2) (layer "F.Cu") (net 1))
 (segment (start 124.206 88.132) (end 123.008 89.33) (width 0.2) (layer "F.Cu") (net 1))
 (segment (start 123.444 82.804) (end 124.206 83.566) (width 0.2) (layer "F.Cu") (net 1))
 (segment (start 109.916 82.362) (end 111.01 82.362) (width 0.2) (layer "F.Cu") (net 1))
 (segment (start 120.4328 91.9052) (end 112.5 91.9052) (width 0.2) (layer "F.Cu") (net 1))
 (segment (start 118.008 84.44) (end 119.634 82.814) (width 0.2) (layer "F.Cu") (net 1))
 (via (at 109.728 82.712) (size 0.6) (drill 0.3) (layers "F.Cu" "B.Cu") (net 1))
 (via (at 109.728 86.614) (size 0.6) (drill 0.3) (layers "F.Cu" "B.Cu") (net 1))
 (segment (start 109.728 82.712) (end 109.728 86.614) (width 0.2) (layer "B.Cu") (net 1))
 (segment (start 123.008 85.605) (end 123.008 88.135) (width 0.2) (layer "F.Cu") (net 5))
 (segment (start 111.6024 91.0076) (end 112.0948 91.5) (width 0.2) (layer "F.Cu") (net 3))
 (segment (start 111.6024 89.4026) (end 111.6024 91.0076) (width 0.2) (layer "F.Cu") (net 3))
 (segment (start 107.442 88.392) (end 108.4526 89.4026) (width 0.2) (layer "F.Cu") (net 3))
 (segment (start 108.4526 89.4026) (end 111.6024 89.4026) (width 0.2) (layer "F.Cu") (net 3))
 (segment (start 113.4559 88.0611) (end 113.4559 90.5441) (width 0.2) (layer "F.Cu") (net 4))
 (segment (start 107.442 85.852) (end 111.2468 85.852) (width 0.2) (layer "F.Cu") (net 4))
 (segment (start 113.4559 90.5441) (end 112.5 91.5) (width 0.2) (layer "F.Cu") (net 4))
 (segment (start 111.2468 85.852) (end 112.7974 87.4026) (width 0.2) (layer "F.Cu") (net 4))
 (segment (start 112.7974 87.4026) (end 113.4559 88.0611) (width 0.2) (layer "F.Cu") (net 4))
 (segment (start 118.008 85.635) (end 115.685 83.312) (width 0.2) (layer "F.Cu") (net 7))
 (segment (start 118.008 85.635) (end 119.313 85.635) (width 0.2) (layer "F.Cu") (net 7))
 (segment (start 119.313 85.635) (end 120.508 84.44) (width 0.2) (layer "F.Cu") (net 7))
 (segment (start 115.685 83.312) (end 113.5 83.312) (width 0.2) (layer "F.Cu") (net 7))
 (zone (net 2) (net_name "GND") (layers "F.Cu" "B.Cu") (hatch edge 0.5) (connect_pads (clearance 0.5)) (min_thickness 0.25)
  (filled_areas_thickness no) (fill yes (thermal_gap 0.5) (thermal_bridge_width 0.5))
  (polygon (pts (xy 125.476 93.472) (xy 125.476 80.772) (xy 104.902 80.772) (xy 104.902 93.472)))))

